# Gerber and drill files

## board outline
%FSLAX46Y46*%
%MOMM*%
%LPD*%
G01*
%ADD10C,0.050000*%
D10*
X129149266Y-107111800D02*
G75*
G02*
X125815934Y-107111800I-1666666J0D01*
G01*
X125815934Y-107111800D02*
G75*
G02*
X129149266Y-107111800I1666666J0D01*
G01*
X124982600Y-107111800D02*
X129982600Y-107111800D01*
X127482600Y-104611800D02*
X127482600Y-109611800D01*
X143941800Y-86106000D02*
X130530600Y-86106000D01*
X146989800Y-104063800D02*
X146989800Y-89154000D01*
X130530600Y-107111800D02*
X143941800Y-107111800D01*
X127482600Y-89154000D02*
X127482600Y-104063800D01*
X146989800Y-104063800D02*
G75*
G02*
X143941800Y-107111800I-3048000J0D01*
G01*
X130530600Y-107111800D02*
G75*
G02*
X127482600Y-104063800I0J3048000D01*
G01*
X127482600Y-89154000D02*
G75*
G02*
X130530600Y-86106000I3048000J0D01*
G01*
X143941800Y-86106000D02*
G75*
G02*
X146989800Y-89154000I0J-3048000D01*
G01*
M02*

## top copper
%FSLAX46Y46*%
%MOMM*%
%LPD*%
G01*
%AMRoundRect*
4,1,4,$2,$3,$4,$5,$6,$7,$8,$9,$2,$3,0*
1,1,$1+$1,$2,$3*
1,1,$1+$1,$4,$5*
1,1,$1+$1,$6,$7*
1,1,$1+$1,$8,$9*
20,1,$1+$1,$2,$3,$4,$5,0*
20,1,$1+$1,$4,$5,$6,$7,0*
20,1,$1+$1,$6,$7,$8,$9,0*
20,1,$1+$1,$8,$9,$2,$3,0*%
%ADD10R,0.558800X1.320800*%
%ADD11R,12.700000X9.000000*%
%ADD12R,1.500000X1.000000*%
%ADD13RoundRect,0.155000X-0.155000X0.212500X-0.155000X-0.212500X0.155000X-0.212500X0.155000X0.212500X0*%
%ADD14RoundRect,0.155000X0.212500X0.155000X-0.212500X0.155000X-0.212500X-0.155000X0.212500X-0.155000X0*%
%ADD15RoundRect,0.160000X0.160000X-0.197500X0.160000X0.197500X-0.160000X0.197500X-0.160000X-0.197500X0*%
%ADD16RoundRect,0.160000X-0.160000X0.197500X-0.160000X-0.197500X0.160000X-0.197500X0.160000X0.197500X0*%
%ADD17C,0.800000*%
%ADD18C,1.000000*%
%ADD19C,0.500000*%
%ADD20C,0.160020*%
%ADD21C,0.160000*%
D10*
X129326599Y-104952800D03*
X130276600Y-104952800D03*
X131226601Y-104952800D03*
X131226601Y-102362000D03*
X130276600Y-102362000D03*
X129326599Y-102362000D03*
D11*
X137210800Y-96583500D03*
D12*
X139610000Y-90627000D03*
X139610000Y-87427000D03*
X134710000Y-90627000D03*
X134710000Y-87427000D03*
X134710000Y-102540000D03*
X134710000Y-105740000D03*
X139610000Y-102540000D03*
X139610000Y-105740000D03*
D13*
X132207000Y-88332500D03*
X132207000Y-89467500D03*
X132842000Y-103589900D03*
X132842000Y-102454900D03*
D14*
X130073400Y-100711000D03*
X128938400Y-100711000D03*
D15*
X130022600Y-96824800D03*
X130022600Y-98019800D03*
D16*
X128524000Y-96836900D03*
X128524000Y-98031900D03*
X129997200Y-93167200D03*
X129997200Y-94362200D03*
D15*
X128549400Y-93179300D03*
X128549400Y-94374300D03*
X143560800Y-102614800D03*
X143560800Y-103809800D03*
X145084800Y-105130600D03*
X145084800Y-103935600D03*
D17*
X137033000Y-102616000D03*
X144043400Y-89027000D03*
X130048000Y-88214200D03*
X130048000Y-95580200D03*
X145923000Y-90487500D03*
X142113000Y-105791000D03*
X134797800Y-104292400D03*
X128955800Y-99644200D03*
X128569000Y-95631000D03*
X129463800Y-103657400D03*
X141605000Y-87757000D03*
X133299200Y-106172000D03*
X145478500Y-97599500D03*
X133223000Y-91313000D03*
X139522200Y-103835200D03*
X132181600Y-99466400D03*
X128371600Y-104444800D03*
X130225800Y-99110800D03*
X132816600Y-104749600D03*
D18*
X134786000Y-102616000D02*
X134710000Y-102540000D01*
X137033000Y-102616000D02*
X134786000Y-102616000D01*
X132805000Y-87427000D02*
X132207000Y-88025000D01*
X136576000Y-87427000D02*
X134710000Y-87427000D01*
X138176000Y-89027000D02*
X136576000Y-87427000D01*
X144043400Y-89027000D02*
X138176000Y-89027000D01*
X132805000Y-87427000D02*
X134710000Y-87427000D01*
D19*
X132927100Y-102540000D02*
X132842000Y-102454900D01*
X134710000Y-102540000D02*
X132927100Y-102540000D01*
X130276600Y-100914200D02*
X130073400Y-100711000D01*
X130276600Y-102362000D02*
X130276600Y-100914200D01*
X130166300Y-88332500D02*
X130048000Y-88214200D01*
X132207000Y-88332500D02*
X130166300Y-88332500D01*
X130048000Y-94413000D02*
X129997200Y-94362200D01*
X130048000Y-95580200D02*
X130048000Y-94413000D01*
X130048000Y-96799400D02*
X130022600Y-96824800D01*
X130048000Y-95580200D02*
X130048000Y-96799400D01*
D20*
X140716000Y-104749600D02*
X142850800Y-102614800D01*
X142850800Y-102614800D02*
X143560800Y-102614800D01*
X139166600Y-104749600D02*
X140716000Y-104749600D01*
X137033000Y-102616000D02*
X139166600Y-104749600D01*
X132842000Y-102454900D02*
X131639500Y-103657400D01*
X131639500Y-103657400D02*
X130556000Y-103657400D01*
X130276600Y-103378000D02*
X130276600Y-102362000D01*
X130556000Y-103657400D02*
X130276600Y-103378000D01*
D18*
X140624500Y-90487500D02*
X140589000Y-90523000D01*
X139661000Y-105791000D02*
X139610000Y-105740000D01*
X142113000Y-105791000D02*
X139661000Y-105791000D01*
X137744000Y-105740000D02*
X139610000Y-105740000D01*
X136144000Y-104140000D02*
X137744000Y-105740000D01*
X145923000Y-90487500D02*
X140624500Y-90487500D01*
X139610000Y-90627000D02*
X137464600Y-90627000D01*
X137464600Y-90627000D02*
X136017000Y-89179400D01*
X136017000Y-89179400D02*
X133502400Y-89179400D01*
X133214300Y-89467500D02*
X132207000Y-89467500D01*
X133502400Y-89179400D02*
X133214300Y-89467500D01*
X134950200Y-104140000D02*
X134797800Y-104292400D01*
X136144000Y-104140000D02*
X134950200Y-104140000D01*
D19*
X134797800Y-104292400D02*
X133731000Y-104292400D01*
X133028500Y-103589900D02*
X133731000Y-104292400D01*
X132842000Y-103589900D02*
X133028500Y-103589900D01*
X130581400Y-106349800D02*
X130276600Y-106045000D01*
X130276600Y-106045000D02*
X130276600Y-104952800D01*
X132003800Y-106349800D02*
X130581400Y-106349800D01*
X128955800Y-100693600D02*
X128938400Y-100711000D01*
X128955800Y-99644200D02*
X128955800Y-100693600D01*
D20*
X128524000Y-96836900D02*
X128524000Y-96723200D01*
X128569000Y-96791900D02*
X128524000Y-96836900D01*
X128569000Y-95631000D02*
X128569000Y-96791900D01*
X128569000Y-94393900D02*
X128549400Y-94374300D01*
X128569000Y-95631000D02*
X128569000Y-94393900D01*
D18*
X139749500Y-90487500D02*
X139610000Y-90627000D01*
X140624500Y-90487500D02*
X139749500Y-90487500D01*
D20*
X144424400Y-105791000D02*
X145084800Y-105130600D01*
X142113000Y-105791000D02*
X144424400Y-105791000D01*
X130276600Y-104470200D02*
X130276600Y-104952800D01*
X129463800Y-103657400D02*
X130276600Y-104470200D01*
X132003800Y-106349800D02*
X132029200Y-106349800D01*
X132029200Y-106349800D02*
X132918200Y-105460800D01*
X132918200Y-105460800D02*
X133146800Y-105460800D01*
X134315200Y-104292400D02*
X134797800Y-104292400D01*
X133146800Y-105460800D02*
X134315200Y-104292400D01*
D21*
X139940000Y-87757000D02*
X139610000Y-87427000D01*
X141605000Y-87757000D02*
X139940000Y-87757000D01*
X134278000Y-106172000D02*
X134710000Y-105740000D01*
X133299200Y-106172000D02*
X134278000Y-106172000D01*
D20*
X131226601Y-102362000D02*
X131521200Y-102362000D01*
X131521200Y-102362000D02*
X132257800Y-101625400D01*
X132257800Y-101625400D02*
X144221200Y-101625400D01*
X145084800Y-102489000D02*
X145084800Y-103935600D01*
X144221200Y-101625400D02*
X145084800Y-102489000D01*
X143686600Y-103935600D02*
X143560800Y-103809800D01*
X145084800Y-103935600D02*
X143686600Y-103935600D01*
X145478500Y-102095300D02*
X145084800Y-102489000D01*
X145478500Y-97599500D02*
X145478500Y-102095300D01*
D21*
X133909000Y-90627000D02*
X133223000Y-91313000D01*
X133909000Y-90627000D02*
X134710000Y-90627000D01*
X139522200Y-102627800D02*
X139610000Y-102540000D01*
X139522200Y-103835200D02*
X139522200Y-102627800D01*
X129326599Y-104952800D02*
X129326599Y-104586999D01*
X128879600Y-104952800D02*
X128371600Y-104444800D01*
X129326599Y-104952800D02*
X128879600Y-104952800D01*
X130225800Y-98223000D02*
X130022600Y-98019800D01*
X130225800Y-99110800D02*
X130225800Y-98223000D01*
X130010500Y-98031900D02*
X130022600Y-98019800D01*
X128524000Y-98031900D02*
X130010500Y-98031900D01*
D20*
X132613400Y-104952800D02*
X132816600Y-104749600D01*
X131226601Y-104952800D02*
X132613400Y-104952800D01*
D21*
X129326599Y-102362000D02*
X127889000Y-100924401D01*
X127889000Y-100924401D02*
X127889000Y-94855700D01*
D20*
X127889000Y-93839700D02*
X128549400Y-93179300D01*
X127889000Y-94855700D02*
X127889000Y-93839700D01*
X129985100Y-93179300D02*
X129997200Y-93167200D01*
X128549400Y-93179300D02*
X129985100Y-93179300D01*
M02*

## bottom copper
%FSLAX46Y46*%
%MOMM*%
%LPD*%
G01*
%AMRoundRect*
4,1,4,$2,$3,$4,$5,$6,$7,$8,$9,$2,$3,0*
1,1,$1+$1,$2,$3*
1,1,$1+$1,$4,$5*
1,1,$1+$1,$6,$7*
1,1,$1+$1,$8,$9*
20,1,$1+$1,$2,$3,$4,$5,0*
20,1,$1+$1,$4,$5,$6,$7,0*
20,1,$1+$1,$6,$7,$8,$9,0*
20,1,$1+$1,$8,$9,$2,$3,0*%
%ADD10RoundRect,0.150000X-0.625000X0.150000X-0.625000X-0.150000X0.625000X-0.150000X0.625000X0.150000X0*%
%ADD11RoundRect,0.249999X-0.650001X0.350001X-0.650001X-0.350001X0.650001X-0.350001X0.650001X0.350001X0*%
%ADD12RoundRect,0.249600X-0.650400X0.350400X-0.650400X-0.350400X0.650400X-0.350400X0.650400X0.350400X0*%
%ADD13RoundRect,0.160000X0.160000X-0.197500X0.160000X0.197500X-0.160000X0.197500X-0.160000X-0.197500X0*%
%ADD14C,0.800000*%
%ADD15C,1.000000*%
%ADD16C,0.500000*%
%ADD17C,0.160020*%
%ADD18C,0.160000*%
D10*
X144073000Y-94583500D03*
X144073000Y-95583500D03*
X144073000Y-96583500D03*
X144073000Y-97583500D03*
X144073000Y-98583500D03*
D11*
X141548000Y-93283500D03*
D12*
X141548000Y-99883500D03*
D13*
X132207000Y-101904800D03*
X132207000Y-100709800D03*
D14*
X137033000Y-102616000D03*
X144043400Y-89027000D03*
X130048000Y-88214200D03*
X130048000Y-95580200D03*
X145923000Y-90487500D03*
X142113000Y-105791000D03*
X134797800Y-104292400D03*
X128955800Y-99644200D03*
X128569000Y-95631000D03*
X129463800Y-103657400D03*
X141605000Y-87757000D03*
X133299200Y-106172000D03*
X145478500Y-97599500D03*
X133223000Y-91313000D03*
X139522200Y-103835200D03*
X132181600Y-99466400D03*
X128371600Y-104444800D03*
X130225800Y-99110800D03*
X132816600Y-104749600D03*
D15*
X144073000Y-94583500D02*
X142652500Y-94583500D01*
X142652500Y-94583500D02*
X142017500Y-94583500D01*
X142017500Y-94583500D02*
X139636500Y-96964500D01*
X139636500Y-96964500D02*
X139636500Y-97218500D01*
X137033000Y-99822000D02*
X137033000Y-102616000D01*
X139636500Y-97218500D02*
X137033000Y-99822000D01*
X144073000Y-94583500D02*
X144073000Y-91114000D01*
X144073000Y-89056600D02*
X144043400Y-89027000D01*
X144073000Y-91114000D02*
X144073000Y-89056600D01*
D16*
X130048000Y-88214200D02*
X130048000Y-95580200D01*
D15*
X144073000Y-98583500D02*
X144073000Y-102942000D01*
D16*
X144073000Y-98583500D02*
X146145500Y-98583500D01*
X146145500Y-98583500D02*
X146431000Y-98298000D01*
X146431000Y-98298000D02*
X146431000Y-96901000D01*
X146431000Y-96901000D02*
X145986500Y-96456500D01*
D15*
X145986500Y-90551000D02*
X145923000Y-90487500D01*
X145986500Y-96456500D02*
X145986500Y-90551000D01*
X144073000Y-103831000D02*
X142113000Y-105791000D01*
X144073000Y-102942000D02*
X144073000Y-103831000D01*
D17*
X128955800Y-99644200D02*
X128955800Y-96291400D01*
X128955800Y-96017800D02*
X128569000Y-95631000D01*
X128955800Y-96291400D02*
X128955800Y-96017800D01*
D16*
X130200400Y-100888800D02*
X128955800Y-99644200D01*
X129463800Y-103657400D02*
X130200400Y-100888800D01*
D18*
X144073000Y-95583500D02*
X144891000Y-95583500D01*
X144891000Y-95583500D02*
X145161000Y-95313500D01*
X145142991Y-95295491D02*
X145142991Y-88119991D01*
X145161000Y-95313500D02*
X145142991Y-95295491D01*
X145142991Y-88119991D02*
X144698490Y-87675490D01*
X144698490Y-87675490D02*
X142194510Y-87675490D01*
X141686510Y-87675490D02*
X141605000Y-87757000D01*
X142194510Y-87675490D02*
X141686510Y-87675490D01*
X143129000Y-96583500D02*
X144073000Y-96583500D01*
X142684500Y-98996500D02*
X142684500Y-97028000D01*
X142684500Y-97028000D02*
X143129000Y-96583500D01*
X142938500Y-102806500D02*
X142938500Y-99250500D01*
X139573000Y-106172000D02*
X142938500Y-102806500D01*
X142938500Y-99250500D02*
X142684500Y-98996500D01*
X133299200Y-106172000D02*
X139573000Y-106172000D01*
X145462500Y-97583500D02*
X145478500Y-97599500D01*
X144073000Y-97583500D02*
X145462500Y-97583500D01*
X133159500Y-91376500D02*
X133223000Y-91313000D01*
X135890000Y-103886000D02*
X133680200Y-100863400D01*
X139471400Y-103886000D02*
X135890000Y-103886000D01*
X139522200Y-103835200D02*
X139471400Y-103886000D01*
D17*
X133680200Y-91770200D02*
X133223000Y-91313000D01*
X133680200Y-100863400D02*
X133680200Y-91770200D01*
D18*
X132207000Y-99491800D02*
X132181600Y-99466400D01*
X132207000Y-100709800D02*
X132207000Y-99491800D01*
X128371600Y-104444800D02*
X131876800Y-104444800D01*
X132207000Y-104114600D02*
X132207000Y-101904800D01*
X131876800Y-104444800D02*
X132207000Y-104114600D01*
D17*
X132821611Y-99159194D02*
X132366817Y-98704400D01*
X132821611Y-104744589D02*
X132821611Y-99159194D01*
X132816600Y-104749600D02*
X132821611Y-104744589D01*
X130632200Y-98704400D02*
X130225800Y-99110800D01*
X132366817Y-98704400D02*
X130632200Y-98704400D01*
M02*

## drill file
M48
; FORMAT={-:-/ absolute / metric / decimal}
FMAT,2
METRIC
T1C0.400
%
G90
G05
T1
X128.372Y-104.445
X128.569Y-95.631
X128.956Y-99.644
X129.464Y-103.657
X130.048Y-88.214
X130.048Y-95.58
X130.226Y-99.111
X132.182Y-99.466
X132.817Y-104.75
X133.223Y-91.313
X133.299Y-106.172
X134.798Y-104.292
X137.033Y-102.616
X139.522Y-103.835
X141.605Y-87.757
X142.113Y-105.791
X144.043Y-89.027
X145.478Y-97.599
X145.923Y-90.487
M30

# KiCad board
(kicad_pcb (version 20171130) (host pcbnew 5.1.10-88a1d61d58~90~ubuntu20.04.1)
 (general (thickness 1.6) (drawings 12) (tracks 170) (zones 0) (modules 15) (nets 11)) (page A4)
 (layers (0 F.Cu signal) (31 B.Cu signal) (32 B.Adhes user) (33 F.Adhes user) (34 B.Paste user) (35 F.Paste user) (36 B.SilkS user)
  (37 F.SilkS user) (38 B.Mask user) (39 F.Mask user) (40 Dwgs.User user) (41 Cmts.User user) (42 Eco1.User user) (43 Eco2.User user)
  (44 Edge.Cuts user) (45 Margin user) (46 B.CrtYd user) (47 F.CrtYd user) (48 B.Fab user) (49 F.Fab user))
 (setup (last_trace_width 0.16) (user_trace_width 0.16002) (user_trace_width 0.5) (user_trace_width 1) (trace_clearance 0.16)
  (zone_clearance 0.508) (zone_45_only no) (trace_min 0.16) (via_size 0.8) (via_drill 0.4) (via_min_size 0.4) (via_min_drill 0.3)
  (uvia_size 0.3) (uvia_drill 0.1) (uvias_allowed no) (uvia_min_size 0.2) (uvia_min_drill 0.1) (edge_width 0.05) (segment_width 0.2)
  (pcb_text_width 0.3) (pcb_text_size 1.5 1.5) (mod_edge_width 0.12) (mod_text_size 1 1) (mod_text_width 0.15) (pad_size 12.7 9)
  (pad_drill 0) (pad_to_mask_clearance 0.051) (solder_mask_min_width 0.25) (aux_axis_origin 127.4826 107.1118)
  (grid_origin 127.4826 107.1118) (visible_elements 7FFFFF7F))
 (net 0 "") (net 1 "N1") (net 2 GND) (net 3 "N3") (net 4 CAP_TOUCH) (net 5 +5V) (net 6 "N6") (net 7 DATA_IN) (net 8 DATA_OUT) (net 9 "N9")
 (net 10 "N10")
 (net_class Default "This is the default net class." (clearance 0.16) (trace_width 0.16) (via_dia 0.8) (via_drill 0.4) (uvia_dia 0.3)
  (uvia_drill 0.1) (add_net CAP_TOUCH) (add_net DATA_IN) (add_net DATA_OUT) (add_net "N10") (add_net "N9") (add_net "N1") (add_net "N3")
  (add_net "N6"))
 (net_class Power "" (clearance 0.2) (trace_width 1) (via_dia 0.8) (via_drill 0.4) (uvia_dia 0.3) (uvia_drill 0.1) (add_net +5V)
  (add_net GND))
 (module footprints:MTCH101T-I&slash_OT (layer F.Cu) (at 130.2766 103.6574 90)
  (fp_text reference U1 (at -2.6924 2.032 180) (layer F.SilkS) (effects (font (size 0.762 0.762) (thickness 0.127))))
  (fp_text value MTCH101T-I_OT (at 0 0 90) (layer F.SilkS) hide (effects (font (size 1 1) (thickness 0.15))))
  (pad 1 smd rect (at -1.2954 -0.950001 90) (size 1.3208 0.5588) (layers F.Cu F.Paste F.Mask) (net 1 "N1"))
  (pad 2 smd rect (at -1.2954 0 90) (size 1.3208 0.5588) (layers F.Cu F.Paste F.Mask) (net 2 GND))
  (pad 3 smd rect (at -1.2954 0.950001 90) (size 1.3208 0.5588) (layers F.Cu F.Paste F.Mask) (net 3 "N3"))
  (pad 4 smd rect (at 1.2954 0.950001 90) (size 1.3208 0.5588) (layers F.Cu F.Paste F.Mask) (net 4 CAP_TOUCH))
  (pad 5 smd rect (at 1.2954 0 90) (size 1.3208 0.5588) (layers F.Cu F.Paste F.Mask) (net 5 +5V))
  (pad 6 smd rect (at 1.2954 -0.950001 90) (size 1.3208 0.5588) (layers F.Cu F.Paste F.Mask) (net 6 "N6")))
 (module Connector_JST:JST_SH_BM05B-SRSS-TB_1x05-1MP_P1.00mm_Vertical (layer B.Cu) (at 142.748 96.5835 270)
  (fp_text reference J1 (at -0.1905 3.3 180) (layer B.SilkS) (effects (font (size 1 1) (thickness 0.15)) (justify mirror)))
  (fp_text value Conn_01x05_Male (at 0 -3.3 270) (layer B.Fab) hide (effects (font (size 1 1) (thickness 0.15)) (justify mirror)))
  (pad 1 smd roundrect (at -2 -1.325 270) (size 0.6 1.55) (layers B.Cu B.Mask) (roundrect_rratio 0.25) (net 5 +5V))
  (pad 2 smd roundrect (at -1 -1.325 270) (size 0.6 1.55) (layers B.Cu B.Mask) (roundrect_rratio 0.25) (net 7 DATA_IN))
  (pad 3 smd roundrect (at 0 -1.325 270) (size 0.6 1.55) (layers B.Cu B.Mask) (roundrect_rratio 0.25) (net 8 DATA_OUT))
  (pad 4 smd roundrect (at 1 -1.325 270) (size 0.6 1.55) (layers B.Cu B.Mask) (roundrect_rratio 0.25) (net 4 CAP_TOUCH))
  (pad 5 smd roundrect (at 2 -1.325 270) (size 0.6 1.55) (layers B.Cu B.Mask) (roundrect_rratio 0.25) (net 2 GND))
  (pad MP smd roundrect (at -3.3 1.2 270) (size 1.2 1.8) (layers B.Cu B.Paste B.Mask) (roundrect_rratio 0.2083325))
  (pad MP smd roundrect (at 3.3 1.2 270) (size 1.2 1.8) (layers B.Cu B.Mask) (roundrect_rratio 0.208)))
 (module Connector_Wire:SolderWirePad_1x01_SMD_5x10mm (layer F.Cu) (at 136.0805 96.647)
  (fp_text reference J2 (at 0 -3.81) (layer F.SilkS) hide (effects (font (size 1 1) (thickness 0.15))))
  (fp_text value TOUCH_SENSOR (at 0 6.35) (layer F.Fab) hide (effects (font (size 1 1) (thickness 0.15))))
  (pad 1 smd rect (at 1.1303 -0.0635) (size 12.7 9) (layers F.Cu F.Mask) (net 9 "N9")))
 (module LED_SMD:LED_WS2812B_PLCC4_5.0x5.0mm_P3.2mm (layer F.Cu) (at 137.16 89.027)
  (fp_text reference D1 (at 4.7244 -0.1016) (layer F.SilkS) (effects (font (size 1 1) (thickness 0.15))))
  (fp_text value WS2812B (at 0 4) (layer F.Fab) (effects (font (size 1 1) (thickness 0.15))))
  (pad 3 smd rect (at 2.45 1.6) (size 1.5 1) (layers F.Cu F.Paste F.Mask) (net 2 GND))
  (pad 4 smd rect (at 2.45 -1.6) (size 1.5 1) (layers F.Cu F.Paste F.Mask) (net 7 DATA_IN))
  (pad 2 smd rect (at -2.45 1.6) (size 1.5 1) (layers F.Cu F.Paste F.Mask) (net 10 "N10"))
  (pad 1 smd rect (at -2.45 -1.6) (size 1.5 1) (layers F.Cu F.Paste F.Mask) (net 5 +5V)))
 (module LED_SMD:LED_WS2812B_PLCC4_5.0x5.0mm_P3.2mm (layer F.Cu) (at 137.16 104.14)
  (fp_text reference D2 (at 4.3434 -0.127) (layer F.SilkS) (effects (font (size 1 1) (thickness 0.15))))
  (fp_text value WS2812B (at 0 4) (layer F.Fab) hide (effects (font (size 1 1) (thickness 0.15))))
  (pad 1 smd rect (at -2.45 -1.6) (size 1.5 1) (layers F.Cu F.Paste F.Mask) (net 5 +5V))
  (pad 2 smd rect (at -2.45 1.6) (size 1.5 1) (layers F.Cu F.Paste F.Mask) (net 8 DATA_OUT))
  (pad 4 smd rect (at 2.45 -1.6) (size 1.5 1) (layers F.Cu F.Paste F.Mask) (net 10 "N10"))
  (pad 3 smd rect (at 2.45 1.6) (size 1.5 1) (layers F.Cu F.Paste F.Mask) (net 2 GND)))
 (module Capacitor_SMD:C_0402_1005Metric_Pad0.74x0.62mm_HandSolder (layer F.Cu) (at 132.207 88.9 270)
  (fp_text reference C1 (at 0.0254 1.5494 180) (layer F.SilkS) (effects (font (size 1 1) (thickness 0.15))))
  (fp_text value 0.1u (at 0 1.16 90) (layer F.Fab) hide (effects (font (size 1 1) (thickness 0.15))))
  (pad 1 smd roundrect (at -0.5675 0 270) (size 0.735 0.62) (layers F.Cu F.Paste F.Mask) (roundrect_rratio 0.25) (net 5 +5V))
  (pad 2 smd roundrect (at 0.5675 0 270) (size 0.735 0.62) (layers F.Cu F.Paste F.Mask) (roundrect_rratio 0.25) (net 2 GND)))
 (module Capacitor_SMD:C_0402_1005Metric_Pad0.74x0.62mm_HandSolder (layer F.Cu) (at 132.842 103.0224 270)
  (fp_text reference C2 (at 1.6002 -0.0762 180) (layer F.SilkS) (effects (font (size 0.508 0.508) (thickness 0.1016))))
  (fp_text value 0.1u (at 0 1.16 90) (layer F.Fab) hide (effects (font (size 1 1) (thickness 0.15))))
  (pad 2 smd roundrect (at 0.5675 0 270) (size 0.735 0.62) (layers F.Cu F.Paste F.Mask) (roundrect_rratio 0.25) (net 2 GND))
  (pad 1 smd roundrect (at -0.5675 0 270) (size 0.735 0.62) (layers F.Cu F.Paste F.Mask) (roundrect_rratio 0.25) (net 5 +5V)))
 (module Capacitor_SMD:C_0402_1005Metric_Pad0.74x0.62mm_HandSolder (layer F.Cu) (at 129.5059 100.711 180)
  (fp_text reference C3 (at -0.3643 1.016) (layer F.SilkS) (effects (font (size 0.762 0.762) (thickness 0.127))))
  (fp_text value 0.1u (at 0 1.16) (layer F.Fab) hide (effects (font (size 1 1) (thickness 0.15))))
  (pad 1 smd roundrect (at -0.5675 0 180) (size 0.735 0.62) (layers F.Cu F.Paste F.Mask) (roundrect_rratio 0.25) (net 5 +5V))
  (pad 2 smd roundrect (at 0.5675 0 180) (size 0.735 0.62) (layers F.Cu F.Paste F.Mask) (roundrect_rratio 0.25) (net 2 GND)))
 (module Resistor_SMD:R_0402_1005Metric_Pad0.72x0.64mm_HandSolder (layer B.Cu) (at 132.207 101.3073 90)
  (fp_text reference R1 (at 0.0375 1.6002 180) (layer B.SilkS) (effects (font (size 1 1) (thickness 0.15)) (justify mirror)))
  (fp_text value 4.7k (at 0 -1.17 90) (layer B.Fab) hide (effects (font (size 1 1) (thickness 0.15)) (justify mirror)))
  (pad 1 smd roundrect (at -0.5975 0 90) (size 0.715 0.64) (layers B.Cu B.Paste B.Mask) (roundrect_rratio 0.25) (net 1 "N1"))
  (pad 2 smd roundrect (at 0.5975 0 90) (size 0.715 0.64) (layers B.Cu B.Paste B.Mask) (roundrect_rratio 0.25) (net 9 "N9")))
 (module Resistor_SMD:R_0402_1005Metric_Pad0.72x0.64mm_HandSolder (layer F.Cu) (at 130.0226 97.4223 90)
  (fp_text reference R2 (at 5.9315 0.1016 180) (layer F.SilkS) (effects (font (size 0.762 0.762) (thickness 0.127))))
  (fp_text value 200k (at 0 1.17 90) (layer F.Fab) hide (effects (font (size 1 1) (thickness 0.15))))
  (pad 2 smd roundrect (at 0.5975 0 90) (size 0.715 0.64) (layers F.Cu F.Paste F.Mask) (roundrect_rratio 0.25) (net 5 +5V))
  (pad 1 smd roundrect (at -0.5975 0 90) (size 0.715 0.64) (layers F.Cu F.Paste F.Mask) (roundrect_rratio 0.25) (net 3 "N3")))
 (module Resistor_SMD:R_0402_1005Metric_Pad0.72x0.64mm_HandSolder (layer F.Cu) (at 128.524 97.4344 270)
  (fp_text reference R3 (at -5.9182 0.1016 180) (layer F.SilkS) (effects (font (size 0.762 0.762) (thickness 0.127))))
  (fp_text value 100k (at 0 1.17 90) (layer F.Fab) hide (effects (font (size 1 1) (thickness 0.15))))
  (pad 1 smd roundrect (at -0.5975 0 270) (size 0.715 0.64) (layers F.Cu F.Paste F.Mask) (roundrect_rratio 0.25) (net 2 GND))
  (pad 2 smd roundrect (at 0.5975 0 270) (size 0.715 0.64) (layers F.Cu F.Paste F.Mask) (roundrect_rratio 0.25) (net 3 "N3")))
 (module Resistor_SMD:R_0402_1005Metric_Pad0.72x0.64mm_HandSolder (layer F.Cu) (at 129.9972 93.7647 270)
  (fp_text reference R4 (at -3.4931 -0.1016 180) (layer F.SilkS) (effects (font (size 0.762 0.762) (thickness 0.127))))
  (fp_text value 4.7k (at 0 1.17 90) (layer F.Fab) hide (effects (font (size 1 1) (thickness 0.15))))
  (pad 1 smd roundrect (at -0.5975 0 270) (size 0.715 0.64) (layers F.Cu F.Paste F.Mask) (roundrect_rratio 0.25) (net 6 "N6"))
  (pad 2 smd roundrect (at 0.5975 0 270) (size 0.715 0.64) (layers F.Cu F.Paste F.Mask) (roundrect_rratio 0.25) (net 5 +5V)))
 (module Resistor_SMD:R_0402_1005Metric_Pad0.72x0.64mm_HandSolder (layer F.Cu) (at 128.5494 93.7768 90)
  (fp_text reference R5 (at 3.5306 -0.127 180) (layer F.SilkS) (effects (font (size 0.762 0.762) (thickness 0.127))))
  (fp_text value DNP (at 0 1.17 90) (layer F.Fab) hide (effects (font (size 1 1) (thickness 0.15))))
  (pad 2 smd roundrect (at 0.5975 0 90) (size 0.715 0.64) (layers F.Cu F.Paste F.Mask) (roundrect_rratio 0.25) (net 6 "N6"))
  (pad 1 smd roundrect (at -0.5975 0 90) (size 0.715 0.64) (layers F.Cu F.Paste F.Mask) (roundrect_rratio 0.25) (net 2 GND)))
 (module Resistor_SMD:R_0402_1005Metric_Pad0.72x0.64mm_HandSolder (layer F.Cu) (at 143.5608 103.2123 90)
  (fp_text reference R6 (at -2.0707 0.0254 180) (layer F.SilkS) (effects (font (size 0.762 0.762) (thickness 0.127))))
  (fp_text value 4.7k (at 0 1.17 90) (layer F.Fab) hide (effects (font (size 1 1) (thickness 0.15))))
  (pad 2 smd roundrect (at 0.5975 0 90) (size 0.715 0.64) (layers F.Cu F.Paste F.Mask) (roundrect_rratio 0.25) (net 5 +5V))
  (pad 1 smd roundrect (at -0.5975 0 90) (size 0.715 0.64) (layers F.Cu F.Paste F.Mask) (roundrect_rratio 0.25) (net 4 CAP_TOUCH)))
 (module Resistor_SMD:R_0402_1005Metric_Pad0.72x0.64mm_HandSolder (layer F.Cu) (at 145.0848 104.5331 90)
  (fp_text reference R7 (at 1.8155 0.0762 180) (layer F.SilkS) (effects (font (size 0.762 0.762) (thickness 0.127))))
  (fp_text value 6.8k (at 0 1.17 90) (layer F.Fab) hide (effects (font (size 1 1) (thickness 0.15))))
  (pad 1 smd roundrect (at -0.5975 0 90) (size 0.715 0.64) (layers F.Cu F.Paste F.Mask) (roundrect_rratio 0.25) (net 2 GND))
  (pad 2 smd roundrect (at 0.5975 0 90) (size 0.715 0.64) (layers F.Cu F.Paste F.Mask) (roundrect_rratio 0.25) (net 4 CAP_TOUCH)))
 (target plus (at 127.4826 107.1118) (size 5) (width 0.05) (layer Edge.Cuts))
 (gr_line (start 143.9418 86.106) (end 130.5306 86.106) (layer Edge.Cuts) (width 0.05))
 (gr_line (start 146.9898 104.0638) (end 146.9898 89.154) (layer Edge.Cuts) (width 0.05))
 (gr_line (start 130.5306 107.1118) (end 143.9418 107.1118) (layer Edge.Cuts) (width 0.05))
 (gr_line (start 127.4826 89.154) (end 127.4826 104.0638) (layer Edge.Cuts) (width 0.05))
 (gr_arc (start 143.9418 104.0638) (end 143.9418 107.1118) (angle -90) (layer Edge.Cuts) (width 0.05))
 (gr_arc (start 130.5306 104.0638) (end 127.4826 104.0638) (angle -90) (layer Edge.Cuts) (width 0.05))
 (gr_arc (start 130.5306 89.154) (end 130.5306 86.106) (angle -90) (layer Edge.Cuts) (width 0.05))
 (gr_arc (start 143.9418 89.154) (end 146.9898 89.154) (angle -90) (layer Edge.Cuts) (width 0.05))
 (segment (start 144.073 94.5835) (end 142.6525 94.5835) (width 1) (layer B.Cu) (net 5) (status 10))
 (segment (start 142.6525 94.5835) (end 142.0175 94.5835) (width 1) (layer B.Cu) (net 5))
 (segment (start 142.0175 94.5835) (end 139.6365 96.9645) (width 1) (layer B.Cu) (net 5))
 (segment (start 139.6365 96.9645) (end 139.6365 97.2185) (width 1) (layer B.Cu) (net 5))
 (via (at 137.033 102.616) (size 0.8) (drill 0.4) (layers F.Cu B.Cu) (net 5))
 (segment (start 137.033 99.822) (end 137.033 102.616) (width 1) (layer B.Cu) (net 5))
 (segment (start 139.6365 97.2185) (end 137.033 99.822) (width 1) (layer B.Cu) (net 5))
 (segment (start 134.786 102.616) (end 134.71 102.54) (width 1) (layer F.Cu) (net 5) (status 30))
 (segment (start 137.033 102.616) (end 134.786 102.616) (width 1) (layer F.Cu) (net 5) (status 20))
 (segment (start 144.073 94.5835) (end 144.073 91.114) (width 1) (layer B.Cu) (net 5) (status 10))
 (segment (start 132.805 87.427) (end 132.207 88.025) (width 1) (layer F.Cu) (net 5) (status 20))
 (via (at 144.0434 89.027) (size 0.8) (drill 0.4) (layers F.Cu B.Cu) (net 5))
 (segment (start 144.073 89.0566) (end 144.0434 89.027) (width 1) (layer B.Cu) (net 5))
 (segment (start 144.073 91.114) (end 144.073 89.0566) (width 1) (layer B.Cu) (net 5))
 (segment (start 136.576 87.427) (end 134.71 87.427) (width 1) (layer F.Cu) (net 5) (status 20))
 (segment (start 138.176 89.027) (end 136.576 87.427) (width 1) (layer F.Cu) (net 5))
 (segment (start 144.0434 89.027) (end 138.176 89.027) (width 1) (layer F.Cu) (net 5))
 (segment (start 132.805 87.427) (end 134.71 87.427) (width 1) (layer F.Cu) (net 5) (status 20))
 (segment (start 132.9271 102.54) (end 132.842 102.4549) (width 0.5) (layer F.Cu) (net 5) (status 30))
 (segment (start 134.71 102.54) (end 132.9271 102.54) (width 0.5) (layer F.Cu) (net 5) (status 30))
 (segment (start 130.2766 100.9142) (end 130.0734 100.711) (width 0.5) (layer F.Cu) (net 5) (status 30))
 (segment (start 130.2766 102.362) (end 130.2766 100.9142) (width 0.5) (layer F.Cu) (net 5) (status 30))
 (via (at 130.048 88.2142) (size 0.8) (drill 0.4) (layers F.Cu B.Cu) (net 5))
 (segment (start 130.1663 88.3325) (end 130.048 88.2142) (width 0.5) (layer F.Cu) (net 5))
 (segment (start 132.207 88.3325) (end 130.1663 88.3325) (width 0.5) (layer F.Cu) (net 5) (status 10))
 (via (at 130.048 95.5802) (size 0.8) (drill 0.4) (layers F.Cu B.Cu) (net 5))
 (segment (start 130.048 88.2142) (end 130.048 95.5802) (width 0.5) (layer B.Cu) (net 5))
 (segment (start 130.048 94.413) (end 129.9972 94.3622) (width 0.5) (layer F.Cu) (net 5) (status 30))
 (segment (start 130.048 95.5802) (end 130.048 94.413) (width 0.5) (layer F.Cu) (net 5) (status 20))
 (segment (start 130.048 96.7994) (end 130.0226 96.8248) (width 0.5) (layer F.Cu) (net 5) (status 30))
 (segment (start 130.048 95.5802) (end 130.048 96.7994) (width 0.5) (layer F.Cu) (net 5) (status 20))
 (segment (start 140.716 104.7496) (end 142.8508 102.6148) (width 0.16002) (layer F.Cu) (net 5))
 (segment (start 142.8508 102.6148) (end 143.5608 102.6148) (width 0.16002) (layer F.Cu) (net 5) (status 20))
 (segment (start 139.1666 104.7496) (end 140.716 104.7496) (width 0.16002) (layer F.Cu) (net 5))
 (segment (start 137.033 102.616) (end 139.1666 104.7496) (width 0.16002) (layer F.Cu) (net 5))
 (segment (start 132.842 102.4549) (end 131.6395 103.6574) (width 0.16002) (layer F.Cu) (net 5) (status 10))
 (segment (start 131.6395 103.6574) (end 130.556 103.6574) (width 0.16002) (layer F.Cu) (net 5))
 (segment (start 130.2766 103.378) (end 130.2766 102.362) (width 0.16002) (layer F.Cu) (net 5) (status 20))
 (segment (start 130.556 103.6574) (end 130.2766 103.378) (width 0.16002) (layer F.Cu) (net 5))
 (segment (start 144.073 98.5835) (end 144.073 102.942) (width 1) (layer B.Cu) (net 2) (status 10))
 (segment (start 144.073 98.5835) (end 146.1455 98.5835) (width 0.5) (layer B.Cu) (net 2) (status 10))
 (segment (start 146.1455 98.5835) (end 146.431 98.298) (width 0.5) (layer B.Cu) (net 2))
 (segment (start 146.431 98.298) (end 146.431 96.901) (width 0.5) (layer B.Cu) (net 2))
 (segment (start 146.431 96.901) (end 145.9865 96.4565) (width 0.5) (layer B.Cu) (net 2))
 (via (at 145.923 90.4875) (size 0.8) (drill 0.4) (layers F.Cu B.Cu) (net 2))
 (segment (start 140.6245 90.4875) (end 140.589 90.523) (width 1) (layer F.Cu) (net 2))
 (segment (start 145.9865 90.551) (end 145.923 90.4875) (width 1) (layer B.Cu) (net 2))
 (segment (start 145.9865 96.4565) (end 145.9865 90.551) (width 1) (layer B.Cu) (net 2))
 (via (at 142.113 105.791) (size 0.8) (drill 0.4) (layers F.Cu B.Cu) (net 2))
 (segment (start 144.073 103.831) (end 142.113 105.791) (width 1) (layer B.Cu) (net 2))
 (segment (start 144.073 102.942) (end 144.073 103.831) (width 1) (layer B.Cu) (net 2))
 (segment (start 139.661 105.791) (end 139.61 105.74) (width 1) (layer F.Cu) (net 2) (status 30))
 (segment (start 142.113 105.791) (end 139.661 105.791) (width 1) (layer F.Cu) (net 2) (status 20))
 (segment (start 137.744 105.74) (end 139.61 105.74) (width 1) (layer F.Cu) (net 2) (status 20))
 (segment (start 136.144 104.14) (end 137.744 105.74) (width 1) (layer F.Cu) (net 2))
 (segment (start 145.923 90.4875) (end 140.6245 90.4875) (width 1) (layer F.Cu) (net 2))
 (segment (start 139.61 90.627) (end 137.4646 90.627) (width 1) (layer F.Cu) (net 2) (status 10))
 (segment (start 137.4646 90.627) (end 136.017 89.1794) (width 1) (layer F.Cu) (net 2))
 (segment (start 136.017 89.1794) (end 133.5024 89.1794) (width 1) (layer F.Cu) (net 2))
 (segment (start 133.2143 89.4675) (end 132.207 89.4675) (width 1) (layer F.Cu) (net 2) (status 20))
 (segment (start 133.5024 89.1794) (end 133.2143 89.4675) (width 1) (layer F.Cu) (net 2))
 (segment (start 134.9502 104.14) (end 134.7978 104.2924) (width 1) (layer F.Cu) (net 2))
 (segment (start 136.144 104.14) (end 134.9502 104.14) (width 1) (layer F.Cu) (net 2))
 (segment (start 134.7978 104.2924) (end 133.731 104.2924) (width 0.5) (layer F.Cu) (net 2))
 (segment (start 133.0285 103.5899) (end 133.731 104.2924) (width 0.5) (layer F.Cu) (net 2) (status 10))
 (segment (start 132.842 103.5899) (end 133.0285 103.5899) (width 0.5) (layer F.Cu) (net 2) (status 30))
 (segment (start 130.5814 106.3498) (end 130.2766 106.045) (width 0.5) (layer F.Cu) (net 2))
 (segment (start 130.2766 106.045) (end 130.2766 104.9528) (width 0.5) (layer F.Cu) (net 2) (status 20))
 (segment (start 132.0038 106.3498) (end 130.5814 106.3498) (width 0.5) (layer F.Cu) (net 2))
 (via (at 134.7978 104.2924) (size 0.8) (drill 0.4) (layers F.Cu B.Cu) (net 2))
 (via (at 128.9558 99.6442) (size 0.8) (drill 0.4) (layers F.Cu B.Cu) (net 2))
 (segment (start 128.9558 100.6936) (end 128.9384 100.711) (width 0.5) (layer F.Cu) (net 2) (status 30))
 (segment (start 128.9558 99.6442) (end 128.9558 100.6936) (width 0.5) (layer F.Cu) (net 2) (status 20))
 (segment (start 128.9558 99.6442) (end 128.9558 96.2914) (width 0.16002) (layer B.Cu) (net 2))
 (segment (start 128.524 96.8369) (end 128.524 96.7232) (width 0.16002) (layer F.Cu) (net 2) (status 30))
 (via (at 128.569 95.631) (size 0.8) (drill 0.4) (layers F.Cu B.Cu) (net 2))
 (segment (start 128.9558 96.0178) (end 128.569 95.631) (width 0.16002) (layer B.Cu) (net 2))
 (segment (start 128.9558 96.2914) (end 128.9558 96.0178) (width 0.16002) (layer B.Cu) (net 2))
 (segment (start 128.569 96.7919) (end 128.524 96.8369) (width 0.16002) (layer F.Cu) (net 2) (status 30))
 (segment (start 128.569 95.631) (end 128.569 96.7919) (width 0.16002) (layer F.Cu) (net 2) (status 20))
 (segment (start 128.569 94.3939) (end 128.5494 94.3743) (width 0.16002) (layer F.Cu) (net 2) (status 30))
 (segment (start 128.569 95.631) (end 128.569 94.3939) (width 0.16002) (layer F.Cu) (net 2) (status 20))
 (segment (start 139.7495 90.4875) (end 139.61 90.627) (width 1) (layer F.Cu) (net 2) (status 30))
 (segment (start 140.6245 90.4875) (end 139.7495 90.4875) (width 1) (layer F.Cu) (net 2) (status 20))
 (segment (start 144.4244 105.791) (end 145.0848 105.1306) (width 0.16002) (layer F.Cu) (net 2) (status 20))
 (segment (start 142.113 105.791) (end 144.4244 105.791) (width 0.16002) (layer F.Cu) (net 2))
 (segment (start 130.2004 100.8888) (end 128.9558 99.6442) (width 0.5) (layer B.Cu) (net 2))
 (segment (start 129.4638 103.6574) (end 130.2004 100.8888) (width 0.5) (layer B.Cu) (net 2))
 (via (at 129.4638 103.6574) (size 0.8) (drill 0.4) (layers F.Cu B.Cu) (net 2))
 (segment (start 130.2766 104.4702) (end 130.2766 104.9528) (width 0.16002) (layer F.Cu) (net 2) (status 30))
 (segment (start 129.4638 103.6574) (end 130.2766 104.4702) (width 0.16002) (layer F.Cu) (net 2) (status 20))
 (segment (start 132.0038 106.3498) (end 132.0292 106.3498) (width 0.16002) (layer F.Cu) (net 2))
 (segment (start 132.0292 106.3498) (end 132.9182 105.4608) (width 0.16002) (layer F.Cu) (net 2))
 (segment (start 132.9182 105.4608) (end 133.1468 105.4608) (width 0.16002) (layer F.Cu) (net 2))
 (segment (start 134.3152 104.2924) (end 134.7978 104.2924) (width 0.16002) (layer F.Cu) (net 2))
 (segment (start 133.1468 105.4608) (end 134.3152 104.2924) (width 0.16002) (layer F.Cu) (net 2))
 (segment (start 144.073 95.5835) (end 144.891 95.5835) (width 0.16) (layer B.Cu) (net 7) (status 10))
 (segment (start 144.891 95.5835) (end 145.161 95.3135) (width 0.16) (layer B.Cu) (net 7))
 (segment (start 145.142991 95.295491) (end 145.142991 88.119991) (width 0.16) (layer B.Cu) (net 7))
 (segment (start 145.161 95.3135) (end 145.142991 95.295491) (width 0.16) (layer B.Cu) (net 7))
 (segment (start 145.142991 88.119991) (end 144.69849 87.67549) (width 0.16) (layer B.Cu) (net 7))
 (segment (start 144.69849 87.67549) (end 142.19451 87.67549) (width 0.16) (layer B.Cu) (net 7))
 (via (at 141.605 87.757) (size 0.8) (drill 0.4) (layers F.Cu B.Cu) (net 7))
 (segment (start 141.68651 87.67549) (end 141.605 87.757) (width 0.16) (layer B.Cu) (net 7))
 (segment (start 142.19451 87.67549) (end 141.68651 87.67549) (width 0.16) (layer B.Cu) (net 7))
 (segment (start 139.94 87.757) (end 139.61 87.427) (width 0.16) (layer F.Cu) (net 7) (status 30))
 (segment (start 141.605 87.757) (end 139.94 87.757) (width 0.16) (layer F.Cu) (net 7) (status 20))
 (segment (start 134.278 106.172) (end 134.71 105.74) (width 0.16) (layer F.Cu) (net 8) (status 30))
 (segment (start 133.2992 106.172) (end 134.278 106.172) (width 0.16) (layer F.Cu) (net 8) (status 20))
 (segment (start 143.129 96.5835) (end 144.073 96.5835) (width 0.16) (layer B.Cu) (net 8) (status 20))
 (segment (start 142.6845 98.9965) (end 142.6845 97.028) (width 0.16) (layer B.Cu) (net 8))
 (segment (start 142.6845 97.028) (end 143.129 96.5835) (width 0.16) (layer B.Cu) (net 8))
 (segment (start 142.9385 102.8065) (end 142.9385 99.2505) (width 0.16) (layer B.Cu) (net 8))
 (segment (start 139.573 106.172) (end 142.9385 102.8065) (width 0.16) (layer B.Cu) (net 8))
 (segment (start 142.9385 99.2505) (end 142.6845 98.9965) (width 0.16) (layer B.Cu) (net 8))
 (segment (start 133.2992 106.172) (end 139.573 106.172) (width 0.16) (layer B.Cu) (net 8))
 (via (at 133.2992 106.172) (size 0.8) (drill 0.4) (layers F.Cu B.Cu) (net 8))
 (via (at 145.4785 97.5995) (size 0.8) (drill 0.4) (layers F.Cu B.Cu) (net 4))
 (segment (start 145.4625 97.5835) (end 145.4785 97.5995) (width 0.16) (layer B.Cu) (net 4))
 (segment (start 144.073 97.5835) (end 145.4625 97.5835) (width 0.16) (layer B.Cu) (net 4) (status 10))
 (segment (start 131.226601 102.362) (end 131.5212 102.362) (width 0.16002) (layer F.Cu) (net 4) (status 10))
 (segment (start 131.5212 102.362) (end 132.2578 101.6254) (width 0.16002) (layer F.Cu) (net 4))
 (segment (start 132.2578 101.6254) (end 144.2212 101.6254) (width 0.16002) (layer F.Cu) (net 4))
 (segment (start 145.0848 102.489) (end 145.0848 103.9356) (width 0.16002) (layer F.Cu) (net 4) (status 20))
 (segment (start 144.2212 101.6254) (end 145.0848 102.489) (width 0.16002) (layer F.Cu) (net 4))
 (segment (start 143.6866 103.9356) (end 143.5608 103.8098) (width 0.16002) (layer F.Cu) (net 4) (status 30))
 (segment (start 145.0848 103.9356) (end 143.6866 103.9356) (width 0.16002) (layer F.Cu) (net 4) (status 30))
 (segment (start 145.4785 102.0953) (end 145.0848 102.489) (width 0.16002) (layer F.Cu) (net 4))
 (segment (start 145.4785 97.5995) (end 145.4785 102.0953) (width 0.16002) (layer F.Cu) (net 4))
 (via (at 133.223 91.313) (size 0.8) (drill 0.4) (layers F.Cu B.Cu) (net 10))
 (segment (start 133.909 90.627) (end 133.223 91.313) (width 0.16) (layer F.Cu) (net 10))
 (via (at 139.5222 103.8352) (size 0.8) (drill 0.4) (layers F.Cu B.Cu) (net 10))
 (segment (start 133.909 90.627) (end 134.71 90.627) (width 0.16) (layer F.Cu) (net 10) (status 20))
 (segment (start 139.5222 102.6278) (end 139.61 102.54) (width 0.16) (layer F.Cu) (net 10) (status 30))
 (segment (start 139.5222 103.8352) (end 139.5222 102.6278) (width 0.16) (layer F.Cu) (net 10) (status 20))
 (segment (start 133.1595 91.3765) (end 133.223 91.313) (width 0.16) (layer B.Cu) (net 10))
 (segment (start 135.89 103.886) (end 133.6802 100.8634) (width 0.16) (layer B.Cu) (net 10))
 (segment (start 139.4714 103.886) (end 135.89 103.886) (width 0.16) (layer B.Cu) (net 10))
 (segment (start 139.5222 103.8352) (end 139.4714 103.886) (width 0.16) (layer B.Cu) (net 10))
 (segment (start 133.6802 91.7702) (end 133.223 91.313) (width 0.16002) (layer B.Cu) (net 10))
 (segment (start 133.6802 100.8634) (end 133.6802 91.7702) (width 0.16002) (layer B.Cu) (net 10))
 (via (at 132.1816 99.4664) (size 0.8) (drill 0.4) (layers F.Cu B.Cu) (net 9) (status 30))
 (segment (start 132.207 99.4918) (end 132.1816 99.4664) (width 0.16) (layer B.Cu) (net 9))
 (segment (start 132.207 100.7098) (end 132.207 99.4918) (width 0.16) (layer B.Cu) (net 9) (status 10))
 (segment (start 129.326599 104.9528) (end 129.326599 104.586999) (width 0.16) (layer F.Cu) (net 1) (status 30))
 (via (at 128.3716 104.4448) (size 0.8) (drill 0.4) (layers F.Cu B.Cu) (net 1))
 (segment (start 128.8796 104.9528) (end 128.3716 104.4448) (width 0.16) (layer F.Cu) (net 1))
 (segment (start 129.326599 104.9528) (end 128.8796 104.9528) (width 0.16) (layer F.Cu) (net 1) (status 10))
 (segment (start 128.3716 104.4448) (end 131.8768 104.4448) (width 0.16) (layer B.Cu) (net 1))
 (segment (start 132.207 104.1146) (end 132.207 101.9048) (width 0.16) (layer B.Cu) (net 1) (status 20))
 (segment (start 131.8768 104.4448) (end 132.207 104.1146) (width 0.16) (layer B.Cu) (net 1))
 (via (at 130.2258 99.1108) (size 0.8) (drill 0.4) (layers F.Cu B.Cu) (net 3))
 (segment (start 130.2258 98.223) (end 130.0226 98.0198) (width 0.16) (layer F.Cu) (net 3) (status 30))
 (segment (start 130.2258 99.1108) (end 130.2258 98.223) (width 0.16) (layer F.Cu) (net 3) (status 20))
 (segment (start 130.0105 98.0319) (end 130.0226 98.0198) (width 0.16) (layer F.Cu) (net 3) (status 30))
 (segment (start 128.524 98.0319) (end 130.0105 98.0319) (width 0.16) (layer F.Cu) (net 3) (status 30))
 (via (at 132.8166 104.7496) (size 0.8) (drill 0.4) (layers F.Cu B.Cu) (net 3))
 (segment (start 132.6134 104.9528) (end 132.8166 104.7496) (width 0.16002) (layer F.Cu) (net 3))
 (segment (start 131.226601 104.9528) (end 132.6134 104.9528) (width 0.16002) (layer F.Cu) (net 3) (status 10))
 (segment (start 132.821611 99.159194) (end 132.366817 98.7044) (width 0.16002) (layer B.Cu) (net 3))
 (segment (start 132.821611 104.744589) (end 132.821611 99.159194) (width 0.16002) (layer B.Cu) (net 3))
 (segment (start 132.8166 104.7496) (end 132.821611 104.744589) (width 0.16002) (layer B.Cu) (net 3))
 (segment (start 130.6322 98.7044) (end 130.2258 99.1108) (width 0.16002) (layer B.Cu) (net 3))
 (segment (start 132.366817 98.7044) (end 130.6322 98.7044) (width 0.16002) (layer B.Cu) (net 3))
 (segment (start 129.326599 102.362) (end 127.889 100.924401) (width 0.16) (layer F.Cu) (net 6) (status 10))
 (segment (start 127.889 100.924401) (end 127.889 94.8557) (width 0.16) (layer F.Cu) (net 6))
 (segment (start 127.889 93.8397) (end 128.5494 93.1793) (width 0.16002) (layer F.Cu) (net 6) (status 20))
 (segment (start 127.889 94.8557) (end 127.889 93.8397) (width 0.16002) (layer F.Cu) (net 6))
 (segment (start 129.9851 93.1793) (end 129.9972 93.1672) (width 0.16002) (layer F.Cu) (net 6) (status 30))
 (segment (start 128.5494 93.1793) (end 129.9851 93.1793) (width 0.16002) (layer F.Cu) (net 6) (status 30)))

